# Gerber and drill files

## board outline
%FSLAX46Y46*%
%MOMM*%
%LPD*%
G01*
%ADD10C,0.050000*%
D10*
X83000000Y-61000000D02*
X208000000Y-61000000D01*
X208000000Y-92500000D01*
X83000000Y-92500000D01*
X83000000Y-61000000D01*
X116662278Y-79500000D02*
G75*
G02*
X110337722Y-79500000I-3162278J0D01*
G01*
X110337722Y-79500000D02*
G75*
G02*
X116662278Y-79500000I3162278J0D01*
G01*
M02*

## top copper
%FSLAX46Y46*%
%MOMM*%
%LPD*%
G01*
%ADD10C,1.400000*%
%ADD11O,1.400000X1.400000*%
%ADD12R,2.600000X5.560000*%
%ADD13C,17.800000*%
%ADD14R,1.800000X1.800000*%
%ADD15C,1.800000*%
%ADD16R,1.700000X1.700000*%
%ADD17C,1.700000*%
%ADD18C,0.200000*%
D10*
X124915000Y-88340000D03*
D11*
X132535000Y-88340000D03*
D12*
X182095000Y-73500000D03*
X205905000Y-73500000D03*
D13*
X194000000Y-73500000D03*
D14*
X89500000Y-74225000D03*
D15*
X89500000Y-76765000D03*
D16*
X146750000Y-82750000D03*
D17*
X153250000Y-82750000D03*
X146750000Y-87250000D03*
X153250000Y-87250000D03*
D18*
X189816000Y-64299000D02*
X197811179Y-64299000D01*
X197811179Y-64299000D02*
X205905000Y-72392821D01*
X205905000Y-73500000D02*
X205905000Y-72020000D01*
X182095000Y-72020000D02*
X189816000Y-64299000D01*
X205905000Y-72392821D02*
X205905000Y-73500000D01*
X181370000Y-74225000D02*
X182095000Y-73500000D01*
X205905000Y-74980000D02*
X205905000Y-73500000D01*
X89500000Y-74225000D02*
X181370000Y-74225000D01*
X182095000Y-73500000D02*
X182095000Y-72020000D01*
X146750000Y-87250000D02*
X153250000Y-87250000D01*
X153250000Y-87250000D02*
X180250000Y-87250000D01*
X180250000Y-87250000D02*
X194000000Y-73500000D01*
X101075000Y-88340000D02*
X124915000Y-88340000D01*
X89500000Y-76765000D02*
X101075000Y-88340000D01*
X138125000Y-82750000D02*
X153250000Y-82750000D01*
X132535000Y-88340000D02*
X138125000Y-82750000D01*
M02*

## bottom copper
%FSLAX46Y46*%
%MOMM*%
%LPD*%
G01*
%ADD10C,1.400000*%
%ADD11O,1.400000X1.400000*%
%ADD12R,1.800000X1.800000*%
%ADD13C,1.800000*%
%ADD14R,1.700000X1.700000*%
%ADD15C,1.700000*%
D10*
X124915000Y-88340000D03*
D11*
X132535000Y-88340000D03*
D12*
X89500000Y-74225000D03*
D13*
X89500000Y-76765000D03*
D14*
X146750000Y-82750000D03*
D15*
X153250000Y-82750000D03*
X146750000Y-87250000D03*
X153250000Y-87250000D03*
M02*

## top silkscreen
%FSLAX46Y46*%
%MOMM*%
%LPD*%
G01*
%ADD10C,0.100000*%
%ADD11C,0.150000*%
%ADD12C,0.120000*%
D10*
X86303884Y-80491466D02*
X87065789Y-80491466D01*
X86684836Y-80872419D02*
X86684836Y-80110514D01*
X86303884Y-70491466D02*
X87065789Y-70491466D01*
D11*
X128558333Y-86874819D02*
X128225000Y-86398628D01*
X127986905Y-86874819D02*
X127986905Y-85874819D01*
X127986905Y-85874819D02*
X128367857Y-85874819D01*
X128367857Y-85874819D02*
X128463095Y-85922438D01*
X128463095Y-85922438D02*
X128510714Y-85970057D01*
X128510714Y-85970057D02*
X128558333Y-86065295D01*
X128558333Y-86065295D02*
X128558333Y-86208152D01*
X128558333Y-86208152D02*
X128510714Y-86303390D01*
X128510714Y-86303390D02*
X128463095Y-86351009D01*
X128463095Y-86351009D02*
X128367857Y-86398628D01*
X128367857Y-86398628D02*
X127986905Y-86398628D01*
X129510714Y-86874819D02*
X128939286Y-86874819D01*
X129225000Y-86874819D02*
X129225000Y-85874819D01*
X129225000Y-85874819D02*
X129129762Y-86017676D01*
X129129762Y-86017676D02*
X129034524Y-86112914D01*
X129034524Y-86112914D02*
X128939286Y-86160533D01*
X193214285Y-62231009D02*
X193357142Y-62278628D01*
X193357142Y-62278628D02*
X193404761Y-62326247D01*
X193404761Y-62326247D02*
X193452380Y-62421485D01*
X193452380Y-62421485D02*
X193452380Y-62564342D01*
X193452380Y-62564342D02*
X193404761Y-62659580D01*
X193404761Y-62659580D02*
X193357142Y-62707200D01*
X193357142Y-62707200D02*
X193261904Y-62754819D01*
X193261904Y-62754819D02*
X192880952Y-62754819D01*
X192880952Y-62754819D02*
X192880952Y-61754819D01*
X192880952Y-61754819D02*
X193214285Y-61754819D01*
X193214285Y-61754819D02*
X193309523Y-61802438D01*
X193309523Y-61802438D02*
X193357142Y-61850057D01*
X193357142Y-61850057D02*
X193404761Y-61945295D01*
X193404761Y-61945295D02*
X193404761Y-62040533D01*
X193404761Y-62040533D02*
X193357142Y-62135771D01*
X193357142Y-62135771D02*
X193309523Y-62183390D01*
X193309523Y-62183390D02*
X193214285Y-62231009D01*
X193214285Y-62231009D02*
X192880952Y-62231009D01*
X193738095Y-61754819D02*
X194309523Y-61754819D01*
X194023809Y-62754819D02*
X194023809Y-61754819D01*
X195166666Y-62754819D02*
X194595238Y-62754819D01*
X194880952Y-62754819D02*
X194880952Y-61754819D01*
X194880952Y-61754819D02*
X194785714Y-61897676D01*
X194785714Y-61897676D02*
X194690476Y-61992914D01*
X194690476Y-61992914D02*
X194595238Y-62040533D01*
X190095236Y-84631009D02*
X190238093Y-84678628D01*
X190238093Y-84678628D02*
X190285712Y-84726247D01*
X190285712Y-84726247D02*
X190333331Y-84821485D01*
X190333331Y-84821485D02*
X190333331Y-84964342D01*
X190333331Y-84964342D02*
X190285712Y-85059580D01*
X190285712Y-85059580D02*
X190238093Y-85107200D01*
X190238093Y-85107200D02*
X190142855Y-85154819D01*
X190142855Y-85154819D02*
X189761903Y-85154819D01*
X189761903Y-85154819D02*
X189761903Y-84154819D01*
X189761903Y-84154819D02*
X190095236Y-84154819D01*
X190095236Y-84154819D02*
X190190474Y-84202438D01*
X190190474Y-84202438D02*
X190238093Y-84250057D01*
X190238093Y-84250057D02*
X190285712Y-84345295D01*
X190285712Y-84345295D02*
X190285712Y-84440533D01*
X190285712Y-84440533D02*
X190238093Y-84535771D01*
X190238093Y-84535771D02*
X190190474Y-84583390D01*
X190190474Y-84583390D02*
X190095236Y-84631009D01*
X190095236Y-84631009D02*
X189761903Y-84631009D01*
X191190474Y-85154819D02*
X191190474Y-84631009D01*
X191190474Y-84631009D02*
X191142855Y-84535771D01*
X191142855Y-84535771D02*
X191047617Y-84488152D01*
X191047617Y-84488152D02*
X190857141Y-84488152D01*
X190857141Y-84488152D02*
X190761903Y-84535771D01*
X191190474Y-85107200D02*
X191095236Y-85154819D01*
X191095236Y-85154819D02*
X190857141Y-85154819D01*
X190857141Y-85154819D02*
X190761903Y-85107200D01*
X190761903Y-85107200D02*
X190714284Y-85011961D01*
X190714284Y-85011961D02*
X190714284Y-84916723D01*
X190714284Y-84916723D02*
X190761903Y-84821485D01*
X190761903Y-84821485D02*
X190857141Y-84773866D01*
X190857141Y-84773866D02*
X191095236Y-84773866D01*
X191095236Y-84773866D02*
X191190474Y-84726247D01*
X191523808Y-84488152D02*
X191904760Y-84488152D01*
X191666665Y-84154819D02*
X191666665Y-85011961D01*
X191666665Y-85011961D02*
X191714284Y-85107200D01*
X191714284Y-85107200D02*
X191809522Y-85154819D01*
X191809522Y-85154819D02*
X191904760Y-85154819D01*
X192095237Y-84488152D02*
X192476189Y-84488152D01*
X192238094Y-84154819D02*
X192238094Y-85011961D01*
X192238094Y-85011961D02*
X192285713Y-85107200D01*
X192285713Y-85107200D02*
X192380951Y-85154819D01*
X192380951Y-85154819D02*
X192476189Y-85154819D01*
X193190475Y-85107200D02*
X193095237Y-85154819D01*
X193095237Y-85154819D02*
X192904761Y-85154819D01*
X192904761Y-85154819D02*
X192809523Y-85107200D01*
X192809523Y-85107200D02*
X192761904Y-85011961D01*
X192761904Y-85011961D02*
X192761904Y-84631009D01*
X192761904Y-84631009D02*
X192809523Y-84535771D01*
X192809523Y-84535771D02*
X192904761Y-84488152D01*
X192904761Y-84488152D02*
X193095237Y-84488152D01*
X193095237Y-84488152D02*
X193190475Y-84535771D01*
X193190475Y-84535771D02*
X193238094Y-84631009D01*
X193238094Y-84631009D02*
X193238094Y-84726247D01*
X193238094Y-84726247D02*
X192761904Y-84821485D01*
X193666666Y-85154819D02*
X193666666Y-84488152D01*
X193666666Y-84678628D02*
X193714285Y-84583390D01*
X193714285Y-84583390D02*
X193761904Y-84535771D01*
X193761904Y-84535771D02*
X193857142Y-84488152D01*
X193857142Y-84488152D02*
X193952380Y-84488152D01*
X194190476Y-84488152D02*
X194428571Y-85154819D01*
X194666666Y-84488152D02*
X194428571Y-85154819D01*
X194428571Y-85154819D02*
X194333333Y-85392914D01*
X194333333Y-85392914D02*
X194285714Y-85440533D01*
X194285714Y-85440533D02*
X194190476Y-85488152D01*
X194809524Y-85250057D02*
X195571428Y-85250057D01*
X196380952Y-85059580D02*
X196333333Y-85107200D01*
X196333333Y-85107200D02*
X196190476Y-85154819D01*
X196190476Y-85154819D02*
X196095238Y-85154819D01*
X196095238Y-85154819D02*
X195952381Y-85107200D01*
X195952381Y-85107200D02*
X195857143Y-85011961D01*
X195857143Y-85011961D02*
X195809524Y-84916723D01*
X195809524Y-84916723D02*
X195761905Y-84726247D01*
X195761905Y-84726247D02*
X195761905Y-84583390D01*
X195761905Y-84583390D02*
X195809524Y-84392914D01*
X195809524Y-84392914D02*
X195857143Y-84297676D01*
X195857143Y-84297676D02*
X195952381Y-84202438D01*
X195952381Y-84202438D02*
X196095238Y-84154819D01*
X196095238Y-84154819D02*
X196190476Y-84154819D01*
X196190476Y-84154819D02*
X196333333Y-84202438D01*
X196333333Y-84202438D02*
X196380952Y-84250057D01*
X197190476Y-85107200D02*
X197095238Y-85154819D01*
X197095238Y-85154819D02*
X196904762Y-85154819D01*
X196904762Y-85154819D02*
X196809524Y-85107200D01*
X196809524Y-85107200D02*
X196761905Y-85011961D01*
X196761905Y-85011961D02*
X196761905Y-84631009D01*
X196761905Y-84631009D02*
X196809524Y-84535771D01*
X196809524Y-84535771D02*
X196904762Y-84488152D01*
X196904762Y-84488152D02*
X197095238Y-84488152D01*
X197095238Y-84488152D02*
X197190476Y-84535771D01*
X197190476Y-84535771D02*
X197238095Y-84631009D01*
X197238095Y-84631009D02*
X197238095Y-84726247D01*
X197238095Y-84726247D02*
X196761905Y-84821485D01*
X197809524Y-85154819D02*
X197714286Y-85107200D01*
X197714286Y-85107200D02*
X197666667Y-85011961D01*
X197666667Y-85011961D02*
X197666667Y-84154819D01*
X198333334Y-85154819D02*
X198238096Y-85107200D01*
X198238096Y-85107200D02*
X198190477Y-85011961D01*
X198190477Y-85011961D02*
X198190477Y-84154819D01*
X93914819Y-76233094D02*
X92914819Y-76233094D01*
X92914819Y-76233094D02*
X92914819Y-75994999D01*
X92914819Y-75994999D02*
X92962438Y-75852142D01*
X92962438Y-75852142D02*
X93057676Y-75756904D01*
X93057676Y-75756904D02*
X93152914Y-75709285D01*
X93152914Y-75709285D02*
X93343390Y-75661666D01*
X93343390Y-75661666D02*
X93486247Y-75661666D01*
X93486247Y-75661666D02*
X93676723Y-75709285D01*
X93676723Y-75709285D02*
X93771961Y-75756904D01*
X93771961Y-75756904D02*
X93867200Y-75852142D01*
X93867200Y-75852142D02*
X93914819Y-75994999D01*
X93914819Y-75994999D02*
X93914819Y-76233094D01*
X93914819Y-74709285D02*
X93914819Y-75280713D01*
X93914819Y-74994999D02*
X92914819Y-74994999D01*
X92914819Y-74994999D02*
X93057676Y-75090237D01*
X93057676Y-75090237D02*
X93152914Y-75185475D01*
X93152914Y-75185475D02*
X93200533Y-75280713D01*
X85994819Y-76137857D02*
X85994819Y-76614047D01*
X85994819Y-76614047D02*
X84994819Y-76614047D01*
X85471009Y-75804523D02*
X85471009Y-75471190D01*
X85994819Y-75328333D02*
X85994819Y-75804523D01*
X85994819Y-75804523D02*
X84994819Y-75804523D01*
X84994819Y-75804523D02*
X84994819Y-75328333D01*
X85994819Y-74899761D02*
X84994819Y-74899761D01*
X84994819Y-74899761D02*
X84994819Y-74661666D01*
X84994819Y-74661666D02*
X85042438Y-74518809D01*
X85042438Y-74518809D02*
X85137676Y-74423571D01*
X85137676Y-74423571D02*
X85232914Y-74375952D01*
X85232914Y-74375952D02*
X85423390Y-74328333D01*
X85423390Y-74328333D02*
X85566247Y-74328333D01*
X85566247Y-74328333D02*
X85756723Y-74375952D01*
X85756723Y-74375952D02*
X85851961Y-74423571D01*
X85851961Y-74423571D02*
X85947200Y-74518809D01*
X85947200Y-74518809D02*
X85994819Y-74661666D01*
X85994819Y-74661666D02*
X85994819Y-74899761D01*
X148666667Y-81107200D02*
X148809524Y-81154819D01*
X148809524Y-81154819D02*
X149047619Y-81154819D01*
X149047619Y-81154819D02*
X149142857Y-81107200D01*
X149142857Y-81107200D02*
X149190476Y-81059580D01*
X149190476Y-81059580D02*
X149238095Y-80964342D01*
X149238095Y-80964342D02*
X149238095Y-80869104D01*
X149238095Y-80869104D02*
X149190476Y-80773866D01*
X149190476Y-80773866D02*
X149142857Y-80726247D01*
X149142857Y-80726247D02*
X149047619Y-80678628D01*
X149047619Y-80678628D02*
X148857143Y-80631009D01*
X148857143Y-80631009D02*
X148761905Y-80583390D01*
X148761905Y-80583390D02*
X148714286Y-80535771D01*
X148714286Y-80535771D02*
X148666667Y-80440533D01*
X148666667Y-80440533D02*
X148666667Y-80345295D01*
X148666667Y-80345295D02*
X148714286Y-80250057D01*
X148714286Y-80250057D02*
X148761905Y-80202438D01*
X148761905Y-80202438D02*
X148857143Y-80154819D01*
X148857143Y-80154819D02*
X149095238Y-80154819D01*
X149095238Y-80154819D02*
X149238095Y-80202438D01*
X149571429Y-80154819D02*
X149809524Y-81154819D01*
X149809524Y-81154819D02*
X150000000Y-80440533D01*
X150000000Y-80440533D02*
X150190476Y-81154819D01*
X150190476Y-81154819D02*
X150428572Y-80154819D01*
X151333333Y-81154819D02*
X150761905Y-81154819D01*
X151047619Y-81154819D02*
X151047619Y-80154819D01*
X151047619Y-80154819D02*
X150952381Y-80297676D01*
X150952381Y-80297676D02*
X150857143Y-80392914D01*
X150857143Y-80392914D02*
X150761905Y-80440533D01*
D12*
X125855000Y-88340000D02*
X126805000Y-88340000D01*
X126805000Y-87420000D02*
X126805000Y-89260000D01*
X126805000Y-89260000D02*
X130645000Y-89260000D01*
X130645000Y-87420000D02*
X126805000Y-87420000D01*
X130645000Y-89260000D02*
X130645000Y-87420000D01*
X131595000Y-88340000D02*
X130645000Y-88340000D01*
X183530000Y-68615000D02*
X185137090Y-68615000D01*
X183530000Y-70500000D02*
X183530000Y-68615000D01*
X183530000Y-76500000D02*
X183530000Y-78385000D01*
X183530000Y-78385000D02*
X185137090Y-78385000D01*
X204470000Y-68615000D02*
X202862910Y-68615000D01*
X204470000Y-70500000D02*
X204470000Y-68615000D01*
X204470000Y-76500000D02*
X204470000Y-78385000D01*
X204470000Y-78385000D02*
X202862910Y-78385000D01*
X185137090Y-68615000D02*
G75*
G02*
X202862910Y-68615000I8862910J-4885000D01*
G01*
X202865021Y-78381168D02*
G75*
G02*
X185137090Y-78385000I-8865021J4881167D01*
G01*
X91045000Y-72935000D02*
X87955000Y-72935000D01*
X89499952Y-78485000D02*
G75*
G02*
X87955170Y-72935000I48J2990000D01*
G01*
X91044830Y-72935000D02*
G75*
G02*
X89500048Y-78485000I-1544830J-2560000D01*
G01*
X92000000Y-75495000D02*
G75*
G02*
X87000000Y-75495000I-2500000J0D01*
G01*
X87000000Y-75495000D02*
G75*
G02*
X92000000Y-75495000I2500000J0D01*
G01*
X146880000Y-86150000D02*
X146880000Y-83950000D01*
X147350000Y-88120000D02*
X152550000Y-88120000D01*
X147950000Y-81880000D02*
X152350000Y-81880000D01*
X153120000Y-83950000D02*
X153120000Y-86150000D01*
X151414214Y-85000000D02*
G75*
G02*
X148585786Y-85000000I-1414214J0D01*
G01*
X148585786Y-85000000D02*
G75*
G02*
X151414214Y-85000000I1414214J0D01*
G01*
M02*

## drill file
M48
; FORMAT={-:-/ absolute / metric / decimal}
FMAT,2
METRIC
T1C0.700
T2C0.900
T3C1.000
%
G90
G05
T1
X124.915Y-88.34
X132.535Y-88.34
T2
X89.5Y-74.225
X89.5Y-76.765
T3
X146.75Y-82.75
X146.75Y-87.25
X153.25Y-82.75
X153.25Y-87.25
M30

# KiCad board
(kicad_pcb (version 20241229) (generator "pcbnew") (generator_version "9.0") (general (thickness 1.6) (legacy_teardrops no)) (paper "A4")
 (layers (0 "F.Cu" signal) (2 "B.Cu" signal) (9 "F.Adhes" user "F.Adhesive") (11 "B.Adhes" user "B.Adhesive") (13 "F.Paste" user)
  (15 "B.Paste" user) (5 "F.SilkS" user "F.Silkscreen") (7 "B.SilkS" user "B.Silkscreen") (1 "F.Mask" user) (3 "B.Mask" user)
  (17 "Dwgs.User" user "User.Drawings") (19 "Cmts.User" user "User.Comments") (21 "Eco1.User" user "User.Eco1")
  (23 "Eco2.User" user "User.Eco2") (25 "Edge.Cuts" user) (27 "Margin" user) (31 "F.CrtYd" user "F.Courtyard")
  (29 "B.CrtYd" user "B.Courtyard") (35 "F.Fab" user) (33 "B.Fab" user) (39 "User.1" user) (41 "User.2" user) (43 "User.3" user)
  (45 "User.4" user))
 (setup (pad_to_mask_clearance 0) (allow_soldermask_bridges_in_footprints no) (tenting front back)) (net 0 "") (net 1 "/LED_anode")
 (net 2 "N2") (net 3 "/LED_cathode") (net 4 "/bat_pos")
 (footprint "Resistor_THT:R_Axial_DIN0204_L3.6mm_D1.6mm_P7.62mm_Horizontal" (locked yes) (layer "F.Cu") (at 124.915 88.34)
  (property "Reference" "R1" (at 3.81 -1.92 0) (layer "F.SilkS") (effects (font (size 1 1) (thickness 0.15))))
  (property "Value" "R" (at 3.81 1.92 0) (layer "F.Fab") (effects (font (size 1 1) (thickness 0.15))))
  (fp_line (start 0.94 0) (end 1.89 0) (stroke (width 0.12) (type solid)) (layer "F.SilkS"))
  (fp_line (start 1.89 -0.92) (end 1.89 0.92) (stroke (width 0.12) (type solid)) (layer "F.SilkS"))
  (fp_line (start 1.89 0.92) (end 5.73 0.92) (stroke (width 0.12) (type solid)) (layer "F.SilkS"))
  (fp_line (start 5.73 -0.92) (end 1.89 -0.92) (stroke (width 0.12) (type solid)) (layer "F.SilkS"))
  (fp_line (start 5.73 0.92) (end 5.73 -0.92) (stroke (width 0.12) (type solid)) (layer "F.SilkS"))
  (fp_line (start 6.68 0) (end 5.73 0) (stroke (width 0.12) (type solid)) (layer "F.SilkS"))
  (pad "1" thru_hole circle (at 0 0) (size 1.4 1.4) (drill 0.7) (layers "*.Cu" "*.Mask") (remove_unused_layers no) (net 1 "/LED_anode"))
  (pad "2" thru_hole oval (at 7.62 0) (size 1.4 1.4) (drill 0.7) (layers "*.Cu" "*.Mask") (remove_unused_layers no) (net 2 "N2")))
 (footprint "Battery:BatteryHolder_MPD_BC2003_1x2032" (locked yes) (layer "F.Cu") (at 194 73.5)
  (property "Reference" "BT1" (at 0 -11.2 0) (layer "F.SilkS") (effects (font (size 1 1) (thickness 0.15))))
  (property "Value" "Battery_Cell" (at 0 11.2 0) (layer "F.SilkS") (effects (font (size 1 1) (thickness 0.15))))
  (fp_line (start -10.47 -4.885) (end -8.86291 -4.885) (stroke (width 0.12) (type solid)) (layer "F.SilkS"))
  (fp_line (start -10.47 -3) (end -10.47 -4.885) (stroke (width 0.12) (type solid)) (layer "F.SilkS"))
  (fp_line (start -10.47 3) (end -10.47 4.885) (stroke (width 0.12) (type solid)) (layer "F.SilkS"))
  (fp_line (start -10.47 4.885) (end -8.86291 4.885) (stroke (width 0.12) (type solid)) (layer "F.SilkS"))
  (fp_line (start 10.47 -4.885) (end 8.86291 -4.885) (stroke (width 0.12) (type solid)) (layer "F.SilkS"))
  (fp_line (start 10.47 -3) (end 10.47 -4.885) (stroke (width 0.12) (type solid)) (layer "F.SilkS"))
  (fp_line (start 10.47 3) (end 10.47 4.885) (stroke (width 0.12) (type solid)) (layer "F.SilkS"))
  (fp_line (start 10.47 4.885) (end 8.86291 4.885) (stroke (width 0.12) (type solid)) (layer "F.SilkS"))
  (fp_arc (start -8.86291 -4.885) (mid 0 -10.12) (end 8.86291 -4.885) (stroke (width 0.12) (type solid)) (layer "F.SilkS"))
  (fp_arc (start 8.865021 4.881168) (mid 0.002187 10.12) (end -8.86291 4.885) (stroke (width 0.12) (type solid)) (layer "F.SilkS"))
  (pad "1" smd rect (at -11.905 0) (size 2.6 5.56) (layers "F.Cu" "F.Mask" "F.Paste") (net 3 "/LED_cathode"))
  (pad "1" smd rect (at 11.905 0) (size 2.6 5.56) (layers "F.Cu" "F.Mask" "F.Paste") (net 3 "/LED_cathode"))
  (pad "2" smd circle (at 0 0) (size 17.8 17.8) (layers "F.Cu" "F.Mask") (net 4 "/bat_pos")))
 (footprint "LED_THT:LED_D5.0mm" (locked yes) (layer "F.Cu") (at 89.5 74.225 -90)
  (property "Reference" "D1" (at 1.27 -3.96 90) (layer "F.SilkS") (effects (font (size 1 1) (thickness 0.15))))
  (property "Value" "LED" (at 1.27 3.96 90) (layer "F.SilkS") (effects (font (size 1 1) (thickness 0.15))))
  (fp_line (start -1.29 -1.545) (end -1.29 1.545) (stroke (width 0.12) (type solid)) (layer "F.SilkS"))
  (fp_arc (start 4.26 0.000048) (mid 2.071756 2.880501) (end -1.29 1.54483) (stroke (width 0.12) (type solid)) (layer "F.SilkS"))
  (fp_arc (start -1.29 -1.54483) (mid 2.071756 -2.880501) (end 4.26 -0.000048) (stroke (width 0.12) (type solid)) (layer "F.SilkS"))
  (fp_circle (center 1.27 0) (end 3.77 0) (stroke (width 0.12) (type solid)) (fill no) (layer "F.SilkS"))
  (pad "1" thru_hole rect (at 0 0 270) (size 1.8 1.8) (drill 0.9) (layers "*.Cu" "*.Mask") (remove_unused_layers no) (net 3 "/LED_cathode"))
  (pad "2" thru_hole circle (at 2.54 0 270) (size 1.8 1.8) (drill 0.9) (layers "*.Cu" "*.Mask") (remove_unused_layers no)
   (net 1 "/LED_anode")))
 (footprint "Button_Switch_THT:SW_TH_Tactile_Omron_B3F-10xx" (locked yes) (layer "F.Cu") (at 146.75 82.75)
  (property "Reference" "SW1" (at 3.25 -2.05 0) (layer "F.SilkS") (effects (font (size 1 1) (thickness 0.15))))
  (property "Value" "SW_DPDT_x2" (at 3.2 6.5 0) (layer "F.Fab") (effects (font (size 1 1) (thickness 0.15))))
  (fp_line (start 0.13 3.4) (end 0.13 1.2) (stroke (width 0.12) (type solid)) (layer "F.SilkS"))
  (fp_line (start 0.6 5.37) (end 5.8 5.37) (stroke (width 0.12) (type solid)) (layer "F.SilkS"))
  (fp_line (start 1.2 -0.87) (end 5.6 -0.87) (stroke (width 0.12) (type solid)) (layer "F.SilkS"))
  (fp_line (start 6.37 1.2) (end 6.37 3.4) (stroke (width 0.12) (type solid)) (layer "F.SilkS"))
  (fp_circle (center 3.25 2.25) (end 4.25 3.25) (stroke (width 0.12) (type solid)) (fill no) (layer "F.SilkS"))
  (pad "1" thru_hole rect (at 0 0) (size 1.7 1.7) (drill 1) (layers "*.Cu" "*.Mask") (remove_unused_layers no) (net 2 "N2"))
  (pad "1" thru_hole circle (at 6.5 0) (size 1.7 1.7) (drill 1) (layers "*.Cu" "*.Mask") (remove_unused_layers no) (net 2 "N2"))
  (pad "2" thru_hole circle (at 0 4.5) (size 1.7 1.7) (drill 1) (layers "*.Cu" "*.Mask") (remove_unused_layers no) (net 4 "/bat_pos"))
  (pad "2" thru_hole circle (at 6.5 4.5) (size 1.7 1.7) (drill 1) (layers "*.Cu" "*.Mask") (remove_unused_layers no) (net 4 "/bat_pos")))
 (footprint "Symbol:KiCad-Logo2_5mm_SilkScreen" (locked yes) (layer "B.Cu") (at 194.5 73.5 180)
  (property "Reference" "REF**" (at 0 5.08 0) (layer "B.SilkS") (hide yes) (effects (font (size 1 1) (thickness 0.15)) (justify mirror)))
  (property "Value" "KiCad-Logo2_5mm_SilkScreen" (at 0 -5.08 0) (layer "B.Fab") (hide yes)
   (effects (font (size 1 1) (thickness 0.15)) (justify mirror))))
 (gr_rect (start 83 61) (end 208 92.5) (stroke (width 0.05) (type default)) (fill no) (locked yes) (layer "Edge.Cuts"))
 (gr_circle (center 113.5 79.5) (end 116.5 80.5) (stroke (width 0.05) (type default)) (fill no) (locked yes) (layer "Edge.Cuts"))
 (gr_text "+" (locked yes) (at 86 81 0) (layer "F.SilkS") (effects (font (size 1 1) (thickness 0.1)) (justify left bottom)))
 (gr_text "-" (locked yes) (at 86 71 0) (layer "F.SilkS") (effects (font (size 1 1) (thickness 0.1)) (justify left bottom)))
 (segment (start 189.816 64.299) (end 197.811179 64.299) (width 0.2) (locked yes) (layer "F.Cu") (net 3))
 (segment (start 197.811179 64.299) (end 205.905 72.392821) (width 0.2) (locked yes) (layer "F.Cu") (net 3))
 (segment (start 205.905 73.5) (end 205.905 72.02) (width 0.2) (locked yes) (layer "F.Cu") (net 3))
 (segment (start 182.095 72.02) (end 189.816 64.299) (width 0.2) (locked yes) (layer "F.Cu") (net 3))
 (segment (start 205.905 72.392821) (end 205.905 73.5) (width 0.2) (locked yes) (layer "F.Cu") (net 3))
 (segment (start 181.37 74.225) (end 182.095 73.5) (width 0.2) (locked yes) (layer "F.Cu") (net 3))
 (segment (start 205.905 74.98) (end 205.905 73.5) (width 0.2) (locked yes) (layer "F.Cu") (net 3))
 (segment (start 89.5 74.225) (end 181.37 74.225) (width 0.2) (locked yes) (layer "F.Cu") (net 3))
 (segment (start 182.095 73.5) (end 182.095 72.02) (width 0.2) (locked yes) (layer "F.Cu") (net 3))
 (segment (start 146.75 87.25) (end 153.25 87.25) (width 0.2) (locked yes) (layer "F.Cu") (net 4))
 (segment (start 153.25 87.25) (end 180.25 87.25) (width 0.2) (locked yes) (layer "F.Cu") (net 4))
 (segment (start 180.25 87.25) (end 194 73.5) (width 0.2) (locked yes) (layer "F.Cu") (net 4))
 (segment (start 101.075 88.34) (end 124.915 88.34) (width 0.2) (locked yes) (layer "F.Cu") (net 1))
 (segment (start 89.5 76.765) (end 101.075 88.34) (width 0.2) (locked yes) (layer "F.Cu") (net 1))
 (segment (start 138.125 82.75) (end 153.25 82.75) (width 0.2) (locked yes) (layer "F.Cu") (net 2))
 (segment (start 132.535 88.34) (end 138.125 82.75) (width 0.2) (locked yes) (layer "F.Cu") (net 2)))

